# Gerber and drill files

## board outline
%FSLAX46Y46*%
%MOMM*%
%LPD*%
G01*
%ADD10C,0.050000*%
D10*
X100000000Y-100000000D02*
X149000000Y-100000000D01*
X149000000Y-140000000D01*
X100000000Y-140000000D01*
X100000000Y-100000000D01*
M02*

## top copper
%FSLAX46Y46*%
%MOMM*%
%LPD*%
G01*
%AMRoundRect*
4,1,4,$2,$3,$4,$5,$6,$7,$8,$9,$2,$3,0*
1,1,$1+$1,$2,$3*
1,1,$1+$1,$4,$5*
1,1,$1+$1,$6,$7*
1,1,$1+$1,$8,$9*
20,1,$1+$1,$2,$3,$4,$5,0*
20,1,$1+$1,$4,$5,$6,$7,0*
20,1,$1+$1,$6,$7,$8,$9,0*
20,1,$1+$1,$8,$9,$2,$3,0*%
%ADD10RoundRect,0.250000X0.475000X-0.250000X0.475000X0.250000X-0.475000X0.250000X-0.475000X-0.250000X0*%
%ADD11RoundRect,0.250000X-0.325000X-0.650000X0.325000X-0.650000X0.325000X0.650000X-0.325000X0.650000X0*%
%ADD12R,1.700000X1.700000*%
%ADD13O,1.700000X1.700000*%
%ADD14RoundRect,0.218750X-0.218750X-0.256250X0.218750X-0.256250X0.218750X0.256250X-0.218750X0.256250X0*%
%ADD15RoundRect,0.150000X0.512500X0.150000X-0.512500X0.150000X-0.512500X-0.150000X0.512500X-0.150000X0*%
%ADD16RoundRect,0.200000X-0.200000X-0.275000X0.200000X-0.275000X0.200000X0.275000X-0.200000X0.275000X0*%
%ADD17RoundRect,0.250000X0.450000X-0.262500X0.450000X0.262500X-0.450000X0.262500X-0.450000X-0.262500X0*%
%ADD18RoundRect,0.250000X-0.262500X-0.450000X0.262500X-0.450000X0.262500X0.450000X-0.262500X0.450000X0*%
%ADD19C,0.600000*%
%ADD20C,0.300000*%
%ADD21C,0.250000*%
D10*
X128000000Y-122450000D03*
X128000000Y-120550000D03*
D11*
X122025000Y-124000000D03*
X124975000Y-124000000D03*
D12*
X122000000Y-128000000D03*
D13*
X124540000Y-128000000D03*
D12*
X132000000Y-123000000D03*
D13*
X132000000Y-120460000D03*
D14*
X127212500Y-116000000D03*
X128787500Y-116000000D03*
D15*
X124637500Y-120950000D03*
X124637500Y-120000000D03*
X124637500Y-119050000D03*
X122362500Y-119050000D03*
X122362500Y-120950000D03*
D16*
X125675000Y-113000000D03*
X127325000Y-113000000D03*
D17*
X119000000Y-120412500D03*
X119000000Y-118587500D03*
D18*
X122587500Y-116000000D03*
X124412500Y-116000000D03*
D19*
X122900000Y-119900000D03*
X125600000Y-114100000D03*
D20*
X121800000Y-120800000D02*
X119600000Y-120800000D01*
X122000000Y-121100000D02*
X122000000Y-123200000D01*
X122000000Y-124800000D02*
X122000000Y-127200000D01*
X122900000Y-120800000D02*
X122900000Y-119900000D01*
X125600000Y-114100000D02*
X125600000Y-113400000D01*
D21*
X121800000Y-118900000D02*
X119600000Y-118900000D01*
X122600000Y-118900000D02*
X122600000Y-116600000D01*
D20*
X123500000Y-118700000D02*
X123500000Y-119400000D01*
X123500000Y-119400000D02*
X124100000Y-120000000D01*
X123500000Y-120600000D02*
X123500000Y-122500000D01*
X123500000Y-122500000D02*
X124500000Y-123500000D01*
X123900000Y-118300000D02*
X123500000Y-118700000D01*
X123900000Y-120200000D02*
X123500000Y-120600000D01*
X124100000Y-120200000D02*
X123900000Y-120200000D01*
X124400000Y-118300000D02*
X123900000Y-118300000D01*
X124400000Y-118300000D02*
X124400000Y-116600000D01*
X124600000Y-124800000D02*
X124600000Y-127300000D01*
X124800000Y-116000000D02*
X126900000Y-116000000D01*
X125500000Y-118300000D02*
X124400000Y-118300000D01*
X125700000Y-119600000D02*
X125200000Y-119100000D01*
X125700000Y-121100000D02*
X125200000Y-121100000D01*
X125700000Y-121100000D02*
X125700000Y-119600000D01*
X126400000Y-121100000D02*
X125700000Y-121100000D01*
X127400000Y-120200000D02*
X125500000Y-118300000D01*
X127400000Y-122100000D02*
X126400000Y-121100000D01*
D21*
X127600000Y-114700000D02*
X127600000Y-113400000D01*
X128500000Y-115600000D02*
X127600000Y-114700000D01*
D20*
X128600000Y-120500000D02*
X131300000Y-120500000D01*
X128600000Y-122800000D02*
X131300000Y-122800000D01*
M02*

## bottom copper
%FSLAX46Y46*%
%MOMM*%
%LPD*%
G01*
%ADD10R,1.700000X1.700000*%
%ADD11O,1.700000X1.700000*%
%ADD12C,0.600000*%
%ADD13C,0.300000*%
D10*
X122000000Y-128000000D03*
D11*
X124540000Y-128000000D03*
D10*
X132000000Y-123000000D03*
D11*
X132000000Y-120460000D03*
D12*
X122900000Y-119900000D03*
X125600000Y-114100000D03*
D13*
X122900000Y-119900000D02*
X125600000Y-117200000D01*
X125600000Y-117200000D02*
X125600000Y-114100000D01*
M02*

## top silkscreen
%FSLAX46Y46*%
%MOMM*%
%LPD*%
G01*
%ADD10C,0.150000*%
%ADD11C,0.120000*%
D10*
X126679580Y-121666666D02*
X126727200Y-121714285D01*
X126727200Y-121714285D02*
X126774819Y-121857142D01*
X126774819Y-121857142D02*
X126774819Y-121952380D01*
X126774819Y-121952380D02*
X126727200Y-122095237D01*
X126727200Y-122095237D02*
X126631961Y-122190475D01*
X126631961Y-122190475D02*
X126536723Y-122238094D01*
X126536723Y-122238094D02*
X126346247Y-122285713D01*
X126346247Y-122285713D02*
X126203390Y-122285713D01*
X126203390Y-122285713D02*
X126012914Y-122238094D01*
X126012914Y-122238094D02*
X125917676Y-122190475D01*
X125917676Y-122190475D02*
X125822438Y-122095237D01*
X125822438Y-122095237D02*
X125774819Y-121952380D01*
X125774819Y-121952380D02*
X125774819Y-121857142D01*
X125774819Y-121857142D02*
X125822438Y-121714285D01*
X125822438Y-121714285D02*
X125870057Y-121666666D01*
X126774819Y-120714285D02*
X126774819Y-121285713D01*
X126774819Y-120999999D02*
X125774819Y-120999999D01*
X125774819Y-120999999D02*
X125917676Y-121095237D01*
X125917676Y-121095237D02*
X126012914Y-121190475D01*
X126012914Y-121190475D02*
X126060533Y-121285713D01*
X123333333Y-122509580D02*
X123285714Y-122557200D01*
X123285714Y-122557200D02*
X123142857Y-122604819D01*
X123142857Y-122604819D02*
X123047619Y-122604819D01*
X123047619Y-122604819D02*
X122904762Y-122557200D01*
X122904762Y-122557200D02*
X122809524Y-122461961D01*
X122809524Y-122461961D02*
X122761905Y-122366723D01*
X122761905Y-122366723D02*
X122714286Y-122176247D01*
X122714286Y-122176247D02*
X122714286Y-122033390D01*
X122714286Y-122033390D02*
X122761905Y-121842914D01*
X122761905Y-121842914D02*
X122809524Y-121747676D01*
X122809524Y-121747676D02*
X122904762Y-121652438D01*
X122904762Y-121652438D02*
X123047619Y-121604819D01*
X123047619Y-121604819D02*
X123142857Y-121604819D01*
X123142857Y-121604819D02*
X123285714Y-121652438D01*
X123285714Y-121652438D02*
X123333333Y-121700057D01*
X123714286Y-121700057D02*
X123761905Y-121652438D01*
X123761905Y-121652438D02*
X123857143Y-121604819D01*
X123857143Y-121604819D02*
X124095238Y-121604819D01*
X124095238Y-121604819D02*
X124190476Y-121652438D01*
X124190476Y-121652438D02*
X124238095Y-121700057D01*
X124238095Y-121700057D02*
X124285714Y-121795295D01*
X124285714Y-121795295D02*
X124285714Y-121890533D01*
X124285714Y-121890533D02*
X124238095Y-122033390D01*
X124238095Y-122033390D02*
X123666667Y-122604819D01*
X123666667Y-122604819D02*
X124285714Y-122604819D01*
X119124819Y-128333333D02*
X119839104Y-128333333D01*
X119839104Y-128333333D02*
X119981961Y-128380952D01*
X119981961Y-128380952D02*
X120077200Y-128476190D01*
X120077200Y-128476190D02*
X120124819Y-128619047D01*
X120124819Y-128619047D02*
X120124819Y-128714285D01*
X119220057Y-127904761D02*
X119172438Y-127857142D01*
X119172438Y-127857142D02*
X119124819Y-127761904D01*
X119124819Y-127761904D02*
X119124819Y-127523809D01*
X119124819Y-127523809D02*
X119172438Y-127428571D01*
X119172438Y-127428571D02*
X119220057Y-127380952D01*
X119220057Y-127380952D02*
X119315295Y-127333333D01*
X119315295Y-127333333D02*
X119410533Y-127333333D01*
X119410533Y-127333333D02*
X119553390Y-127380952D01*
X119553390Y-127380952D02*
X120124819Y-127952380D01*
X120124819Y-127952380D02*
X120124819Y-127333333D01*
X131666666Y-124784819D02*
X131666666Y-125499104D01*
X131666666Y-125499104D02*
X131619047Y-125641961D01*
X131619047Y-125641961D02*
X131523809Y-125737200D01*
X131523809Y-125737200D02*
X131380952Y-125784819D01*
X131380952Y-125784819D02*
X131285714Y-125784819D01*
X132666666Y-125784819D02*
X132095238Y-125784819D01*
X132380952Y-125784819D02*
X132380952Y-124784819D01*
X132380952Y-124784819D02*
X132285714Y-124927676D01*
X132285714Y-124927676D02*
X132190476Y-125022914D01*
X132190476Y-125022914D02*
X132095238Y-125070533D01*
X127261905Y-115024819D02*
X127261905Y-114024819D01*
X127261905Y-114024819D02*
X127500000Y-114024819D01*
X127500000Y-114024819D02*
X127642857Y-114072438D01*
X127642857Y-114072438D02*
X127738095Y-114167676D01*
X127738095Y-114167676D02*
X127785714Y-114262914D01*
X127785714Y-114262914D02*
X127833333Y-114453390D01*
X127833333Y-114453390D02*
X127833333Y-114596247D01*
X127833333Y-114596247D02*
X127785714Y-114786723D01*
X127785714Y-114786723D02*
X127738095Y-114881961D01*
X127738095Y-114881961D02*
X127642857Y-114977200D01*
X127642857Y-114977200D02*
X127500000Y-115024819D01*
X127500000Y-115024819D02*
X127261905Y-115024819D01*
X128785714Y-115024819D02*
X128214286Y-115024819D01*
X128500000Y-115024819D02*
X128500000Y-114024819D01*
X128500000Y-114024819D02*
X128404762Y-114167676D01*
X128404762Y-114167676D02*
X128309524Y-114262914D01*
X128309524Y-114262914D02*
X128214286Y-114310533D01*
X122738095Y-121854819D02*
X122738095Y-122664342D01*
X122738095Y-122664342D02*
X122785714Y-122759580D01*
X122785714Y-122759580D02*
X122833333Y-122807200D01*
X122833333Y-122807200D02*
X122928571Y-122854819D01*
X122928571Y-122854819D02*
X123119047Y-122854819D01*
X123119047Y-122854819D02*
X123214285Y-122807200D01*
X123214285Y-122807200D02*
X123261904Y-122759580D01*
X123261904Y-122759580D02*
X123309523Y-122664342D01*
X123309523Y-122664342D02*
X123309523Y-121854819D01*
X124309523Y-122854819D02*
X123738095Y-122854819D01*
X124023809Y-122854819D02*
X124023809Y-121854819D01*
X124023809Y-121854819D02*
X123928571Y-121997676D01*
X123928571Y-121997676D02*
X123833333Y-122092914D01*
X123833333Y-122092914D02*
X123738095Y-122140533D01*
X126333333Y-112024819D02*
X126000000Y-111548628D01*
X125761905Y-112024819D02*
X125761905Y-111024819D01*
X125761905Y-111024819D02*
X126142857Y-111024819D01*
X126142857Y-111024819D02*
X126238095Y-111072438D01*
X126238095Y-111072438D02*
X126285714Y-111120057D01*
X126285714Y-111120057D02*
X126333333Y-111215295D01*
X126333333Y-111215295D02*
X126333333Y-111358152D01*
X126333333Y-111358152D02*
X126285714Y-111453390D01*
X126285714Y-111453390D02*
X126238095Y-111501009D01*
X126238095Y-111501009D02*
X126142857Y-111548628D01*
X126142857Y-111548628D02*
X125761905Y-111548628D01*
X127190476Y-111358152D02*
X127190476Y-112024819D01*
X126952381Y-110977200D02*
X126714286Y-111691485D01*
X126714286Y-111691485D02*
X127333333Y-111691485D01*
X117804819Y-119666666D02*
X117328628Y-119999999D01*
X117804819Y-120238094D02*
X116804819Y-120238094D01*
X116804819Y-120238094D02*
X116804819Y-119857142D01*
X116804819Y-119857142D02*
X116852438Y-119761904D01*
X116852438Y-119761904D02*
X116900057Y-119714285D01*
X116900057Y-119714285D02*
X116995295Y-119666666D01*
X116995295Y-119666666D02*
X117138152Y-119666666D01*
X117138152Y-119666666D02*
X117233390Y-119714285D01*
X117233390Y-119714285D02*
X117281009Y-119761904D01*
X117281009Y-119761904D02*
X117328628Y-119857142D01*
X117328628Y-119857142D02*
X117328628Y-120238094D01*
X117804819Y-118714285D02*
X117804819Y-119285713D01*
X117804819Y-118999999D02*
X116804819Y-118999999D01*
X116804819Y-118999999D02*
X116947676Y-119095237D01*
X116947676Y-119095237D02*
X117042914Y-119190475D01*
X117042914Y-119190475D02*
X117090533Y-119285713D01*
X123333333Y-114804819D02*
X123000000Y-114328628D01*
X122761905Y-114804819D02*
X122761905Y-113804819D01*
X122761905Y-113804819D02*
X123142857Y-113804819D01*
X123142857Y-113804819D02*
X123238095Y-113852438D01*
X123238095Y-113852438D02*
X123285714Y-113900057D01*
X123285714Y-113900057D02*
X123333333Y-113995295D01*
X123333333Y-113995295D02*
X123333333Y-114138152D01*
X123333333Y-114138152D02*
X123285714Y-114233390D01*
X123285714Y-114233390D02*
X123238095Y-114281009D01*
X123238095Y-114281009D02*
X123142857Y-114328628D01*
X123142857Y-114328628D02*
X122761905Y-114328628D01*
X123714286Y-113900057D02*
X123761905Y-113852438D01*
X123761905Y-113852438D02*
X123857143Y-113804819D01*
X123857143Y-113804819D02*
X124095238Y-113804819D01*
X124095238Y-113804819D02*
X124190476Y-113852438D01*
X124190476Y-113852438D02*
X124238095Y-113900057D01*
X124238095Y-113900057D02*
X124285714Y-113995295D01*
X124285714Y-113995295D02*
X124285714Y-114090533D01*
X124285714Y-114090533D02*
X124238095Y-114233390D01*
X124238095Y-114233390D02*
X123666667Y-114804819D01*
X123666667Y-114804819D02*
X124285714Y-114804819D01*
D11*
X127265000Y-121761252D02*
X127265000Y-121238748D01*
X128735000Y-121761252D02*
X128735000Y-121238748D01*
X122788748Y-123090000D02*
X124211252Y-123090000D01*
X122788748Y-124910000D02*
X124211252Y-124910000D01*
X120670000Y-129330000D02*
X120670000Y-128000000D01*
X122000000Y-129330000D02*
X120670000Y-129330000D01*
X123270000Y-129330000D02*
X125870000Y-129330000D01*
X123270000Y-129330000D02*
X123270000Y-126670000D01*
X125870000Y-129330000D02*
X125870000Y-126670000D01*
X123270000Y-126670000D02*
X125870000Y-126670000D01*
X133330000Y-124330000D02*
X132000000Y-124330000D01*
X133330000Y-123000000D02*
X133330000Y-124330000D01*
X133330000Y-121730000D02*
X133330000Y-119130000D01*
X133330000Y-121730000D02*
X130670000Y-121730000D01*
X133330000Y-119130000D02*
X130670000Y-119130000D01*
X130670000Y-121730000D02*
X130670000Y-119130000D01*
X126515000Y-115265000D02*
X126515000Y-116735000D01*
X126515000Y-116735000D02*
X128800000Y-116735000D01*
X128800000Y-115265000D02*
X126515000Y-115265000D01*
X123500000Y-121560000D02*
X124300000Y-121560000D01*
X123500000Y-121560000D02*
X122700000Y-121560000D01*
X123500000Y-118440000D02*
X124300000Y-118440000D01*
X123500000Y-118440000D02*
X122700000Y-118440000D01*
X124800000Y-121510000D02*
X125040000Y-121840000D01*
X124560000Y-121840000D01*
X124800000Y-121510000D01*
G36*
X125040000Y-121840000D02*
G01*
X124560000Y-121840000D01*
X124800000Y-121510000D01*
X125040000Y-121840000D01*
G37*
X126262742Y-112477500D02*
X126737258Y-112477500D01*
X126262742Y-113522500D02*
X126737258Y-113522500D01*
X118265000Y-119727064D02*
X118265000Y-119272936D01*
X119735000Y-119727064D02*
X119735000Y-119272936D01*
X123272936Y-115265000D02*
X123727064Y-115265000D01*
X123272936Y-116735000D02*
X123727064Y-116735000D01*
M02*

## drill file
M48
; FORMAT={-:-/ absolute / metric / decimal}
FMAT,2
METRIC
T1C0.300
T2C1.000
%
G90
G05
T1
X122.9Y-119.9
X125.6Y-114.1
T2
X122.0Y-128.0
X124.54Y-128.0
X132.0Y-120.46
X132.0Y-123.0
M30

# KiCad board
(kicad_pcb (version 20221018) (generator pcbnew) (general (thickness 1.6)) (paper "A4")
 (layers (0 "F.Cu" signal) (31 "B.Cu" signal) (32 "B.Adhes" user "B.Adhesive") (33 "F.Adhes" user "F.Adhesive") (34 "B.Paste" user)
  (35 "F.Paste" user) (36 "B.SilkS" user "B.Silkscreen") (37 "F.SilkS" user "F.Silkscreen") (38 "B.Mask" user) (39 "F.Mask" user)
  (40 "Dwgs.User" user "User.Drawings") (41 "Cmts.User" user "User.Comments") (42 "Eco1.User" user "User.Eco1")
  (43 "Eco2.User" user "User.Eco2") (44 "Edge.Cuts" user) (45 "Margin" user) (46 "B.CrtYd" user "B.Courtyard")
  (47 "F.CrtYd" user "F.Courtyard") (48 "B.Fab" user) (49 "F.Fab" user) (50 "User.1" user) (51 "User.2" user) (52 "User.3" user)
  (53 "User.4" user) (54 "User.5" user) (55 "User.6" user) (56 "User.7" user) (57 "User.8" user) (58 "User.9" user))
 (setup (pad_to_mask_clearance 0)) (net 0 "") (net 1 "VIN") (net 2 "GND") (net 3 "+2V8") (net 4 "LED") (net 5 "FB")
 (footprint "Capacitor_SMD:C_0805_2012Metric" (layer "F.Cu") (at 128 121.5 90)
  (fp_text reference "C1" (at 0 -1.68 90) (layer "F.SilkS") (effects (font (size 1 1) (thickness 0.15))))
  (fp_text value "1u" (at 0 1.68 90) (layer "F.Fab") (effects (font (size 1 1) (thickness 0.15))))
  (fp_line (start -0.261252 -0.735) (end 0.261252 -0.735) (stroke (width 0.12) (type solid)) (layer "F.SilkS"))
  (fp_line (start -0.261252 0.735) (end 0.261252 0.735) (stroke (width 0.12) (type solid)) (layer "F.SilkS"))
  (pad "1" smd roundrect (at -0.95 0 90) (size 1 1.45) (layers "F.Cu" "F.Paste" "F.Mask") (roundrect_rratio 0.25) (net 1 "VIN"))
  (pad "2" smd roundrect (at 0.95 0 90) (size 1 1.45) (layers "F.Cu" "F.Paste" "F.Mask") (roundrect_rratio 0.25) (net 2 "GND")))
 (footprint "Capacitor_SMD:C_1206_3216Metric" (layer "F.Cu") (at 123.5 124)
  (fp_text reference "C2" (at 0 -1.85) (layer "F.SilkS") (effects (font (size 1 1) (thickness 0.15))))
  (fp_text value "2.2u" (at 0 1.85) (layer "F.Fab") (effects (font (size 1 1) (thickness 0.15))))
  (fp_line (start -0.711252 -0.91) (end 0.711252 -0.91) (stroke (width 0.12) (type solid)) (layer "F.SilkS"))
  (fp_line (start -0.711252 0.91) (end 0.711252 0.91) (stroke (width 0.12) (type solid)) (layer "F.SilkS"))
  (pad "1" smd roundrect (at -1.475 0) (size 1.15 1.8) (layers "F.Cu" "F.Paste" "F.Mask") (roundrect_rratio 0.217391) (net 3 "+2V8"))
  (pad "2" smd roundrect (at 1.475 0) (size 1.15 1.8) (layers "F.Cu" "F.Paste" "F.Mask") (roundrect_rratio 0.217391) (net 2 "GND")))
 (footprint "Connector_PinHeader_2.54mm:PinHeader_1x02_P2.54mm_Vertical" (layer "F.Cu") (at 122 128 90)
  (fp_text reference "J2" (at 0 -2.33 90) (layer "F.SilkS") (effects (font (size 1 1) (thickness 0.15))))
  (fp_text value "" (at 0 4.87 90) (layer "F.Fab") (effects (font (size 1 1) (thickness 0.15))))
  (fp_line (start -1.33 -1.33) (end 0 -1.33) (stroke (width 0.12) (type solid)) (layer "F.SilkS"))
  (fp_line (start -1.33 0) (end -1.33 -1.33) (stroke (width 0.12) (type solid)) (layer "F.SilkS"))
  (fp_line (start -1.33 1.27) (end -1.33 3.87) (stroke (width 0.12) (type solid)) (layer "F.SilkS"))
  (fp_line (start -1.33 1.27) (end 1.33 1.27) (stroke (width 0.12) (type solid)) (layer "F.SilkS"))
  (fp_line (start -1.33 3.87) (end 1.33 3.87) (stroke (width 0.12) (type solid)) (layer "F.SilkS"))
  (fp_line (start 1.33 1.27) (end 1.33 3.87) (stroke (width 0.12) (type solid)) (layer "F.SilkS"))
  (pad "1" thru_hole rect (at 0 0 90) (size 1.7 1.7) (drill 1) (layers "*.Cu" "*.Mask") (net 3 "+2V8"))
  (pad "2" thru_hole oval (at 0 2.54 90) (size 1.7 1.7) (drill 1) (layers "*.Cu" "*.Mask") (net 2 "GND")))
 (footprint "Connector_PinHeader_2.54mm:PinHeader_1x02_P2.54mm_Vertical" (layer "F.Cu") (at 132 123 180)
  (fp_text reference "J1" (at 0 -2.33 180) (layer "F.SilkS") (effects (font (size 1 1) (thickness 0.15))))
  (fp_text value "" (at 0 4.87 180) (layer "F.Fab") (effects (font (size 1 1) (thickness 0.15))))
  (fp_line (start -1.33 -1.33) (end 0 -1.33) (stroke (width 0.12) (type solid)) (layer "F.SilkS"))
  (fp_line (start -1.33 0) (end -1.33 -1.33) (stroke (width 0.12) (type solid)) (layer "F.SilkS"))
  (fp_line (start -1.33 1.27) (end -1.33 3.87) (stroke (width 0.12) (type solid)) (layer "F.SilkS"))
  (fp_line (start -1.33 1.27) (end 1.33 1.27) (stroke (width 0.12) (type solid)) (layer "F.SilkS"))
  (fp_line (start -1.33 3.87) (end 1.33 3.87) (stroke (width 0.12) (type solid)) (layer "F.SilkS"))
  (fp_line (start 1.33 1.27) (end 1.33 3.87) (stroke (width 0.12) (type solid)) (layer "F.SilkS"))
  (pad "1" thru_hole rect (at 0 0 180) (size 1.7 1.7) (drill 1) (layers "*.Cu" "*.Mask") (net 1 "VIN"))
  (pad "2" thru_hole oval (at 0 2.54 180) (size 1.7 1.7) (drill 1) (layers "*.Cu" "*.Mask") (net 2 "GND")))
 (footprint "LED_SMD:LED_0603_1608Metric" (layer "F.Cu") (at 128 116)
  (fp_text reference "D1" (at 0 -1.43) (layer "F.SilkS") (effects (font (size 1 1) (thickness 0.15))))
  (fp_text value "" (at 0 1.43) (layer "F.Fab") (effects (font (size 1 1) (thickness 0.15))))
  (fp_line (start -1.485 -0.735) (end -1.485 0.735) (stroke (width 0.12) (type solid)) (layer "F.SilkS"))
  (fp_line (start -1.485 0.735) (end 0.8 0.735) (stroke (width 0.12) (type solid)) (layer "F.SilkS"))
  (fp_line (start 0.8 -0.735) (end -1.485 -0.735) (stroke (width 0.12) (type solid)) (layer "F.SilkS"))
  (pad "1" smd roundrect (at -0.7875 0) (size 0.875 0.95) (layers "F.Cu" "F.Paste" "F.Mask") (roundrect_rratio 0.25) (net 2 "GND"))
  (pad "2" smd roundrect (at 0.7875 0) (size 0.875 0.95) (layers "F.Cu" "F.Paste" "F.Mask") (roundrect_rratio 0.25) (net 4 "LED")))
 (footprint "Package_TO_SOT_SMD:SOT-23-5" (layer "F.Cu") (at 123.5 120 180)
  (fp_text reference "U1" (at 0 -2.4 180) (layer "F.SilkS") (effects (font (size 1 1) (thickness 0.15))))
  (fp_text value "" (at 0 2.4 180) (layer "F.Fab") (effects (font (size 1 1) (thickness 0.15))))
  (fp_line (start 0 -1.56) (end -0.8 -1.56) (stroke (width 0.12) (type solid)) (layer "F.SilkS"))
  (fp_line (start 0 -1.56) (end 0.8 -1.56) (stroke (width 0.12) (type solid)) (layer "F.SilkS"))
  (fp_line (start 0 1.56) (end -0.8 1.56) (stroke (width 0.12) (type solid)) (layer "F.SilkS"))
  (fp_line (start 0 1.56) (end 0.8 1.56) (stroke (width 0.12) (type solid)) (layer "F.SilkS"))
  (fp_poly
   (pts (xy -1.3 -1.51) (xy -1.54 -1.84) (xy -1.06 -1.84) (xy -1.3 -1.51)) (stroke (width 0.12) (type solid)) (fill solid) (layer "F.SilkS"))
  (pad "1" smd roundrect (at -1.1375 -0.95 180) (size 1.325 0.6) (layers "F.Cu" "F.Paste" "F.Mask") (roundrect_rratio 0.25) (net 1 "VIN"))
  (pad "2" smd roundrect (at -1.1375 0 180) (size 1.325 0.6) (layers "F.Cu" "F.Paste" "F.Mask") (roundrect_rratio 0.25) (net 2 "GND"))
  (pad "3" smd roundrect (at -1.1375 0.95 180) (size 1.325 0.6) (layers "F.Cu" "F.Paste" "F.Mask") (roundrect_rratio 0.25) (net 1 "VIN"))
  (pad "4" smd roundrect (at 1.1375 0.95 180) (size 1.325 0.6) (layers "F.Cu" "F.Paste" "F.Mask") (roundrect_rratio 0.25) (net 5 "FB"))
  (pad "5" smd roundrect (at 1.1375 -0.95 180) (size 1.325 0.6) (layers "F.Cu" "F.Paste" "F.Mask") (roundrect_rratio 0.25) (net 3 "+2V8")))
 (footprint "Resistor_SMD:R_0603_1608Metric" (layer "F.Cu") (at 126.5 113)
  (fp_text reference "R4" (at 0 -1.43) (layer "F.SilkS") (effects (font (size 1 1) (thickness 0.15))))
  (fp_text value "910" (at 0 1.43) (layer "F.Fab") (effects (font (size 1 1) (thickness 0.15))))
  (fp_line (start -0.237258 -0.5225) (end 0.237258 -0.5225) (stroke (width 0.12) (type solid)) (layer "F.SilkS"))
  (fp_line (start -0.237258 0.5225) (end 0.237258 0.5225) (stroke (width 0.12) (type solid)) (layer "F.SilkS"))
  (pad "1" smd roundrect (at -0.825 0) (size 0.8 0.95) (layers "F.Cu" "F.Paste" "F.Mask") (roundrect_rratio 0.25) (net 3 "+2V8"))
  (pad "2" smd roundrect (at 0.825 0) (size 0.8 0.95) (layers "F.Cu" "F.Paste" "F.Mask") (roundrect_rratio 0.25) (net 4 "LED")))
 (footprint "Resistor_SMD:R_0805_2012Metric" (layer "F.Cu") (at 119 119.5 90)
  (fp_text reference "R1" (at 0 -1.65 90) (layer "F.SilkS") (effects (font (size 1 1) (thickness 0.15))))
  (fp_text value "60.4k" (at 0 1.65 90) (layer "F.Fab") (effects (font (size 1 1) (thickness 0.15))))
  (fp_line (start -0.227064 -0.735) (end 0.227064 -0.735) (stroke (width 0.12) (type solid)) (layer "F.SilkS"))
  (fp_line (start -0.227064 0.735) (end 0.227064 0.735) (stroke (width 0.12) (type solid)) (layer "F.SilkS"))
  (pad "1" smd roundrect (at -0.9125 0 90) (size 1.025 1.4) (layers "F.Cu" "F.Paste" "F.Mask") (roundrect_rratio 0.243902) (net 3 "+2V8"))
  (pad "2" smd roundrect (at 0.9125 0 90) (size 1.025 1.4) (layers "F.Cu" "F.Paste" "F.Mask") (roundrect_rratio 0.243902) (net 5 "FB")))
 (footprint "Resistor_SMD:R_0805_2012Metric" (layer "F.Cu") (at 123.5 116)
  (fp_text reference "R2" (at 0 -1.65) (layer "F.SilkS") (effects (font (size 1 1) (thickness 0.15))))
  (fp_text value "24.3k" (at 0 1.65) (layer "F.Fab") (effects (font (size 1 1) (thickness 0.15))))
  (fp_line (start -0.227064 -0.735) (end 0.227064 -0.735) (stroke (width 0.12) (type solid)) (layer "F.SilkS"))
  (fp_line (start -0.227064 0.735) (end 0.227064 0.735) (stroke (width 0.12) (type solid)) (layer "F.SilkS"))
  (pad "1" smd roundrect (at -0.9125 0) (size 1.025 1.4) (layers "F.Cu" "F.Paste" "F.Mask") (roundrect_rratio 0.243902) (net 5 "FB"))
  (pad "2" smd roundrect (at 0.9125 0) (size 1.025 1.4) (layers "F.Cu" "F.Paste" "F.Mask") (roundrect_rratio 0.243902) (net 2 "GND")))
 (gr_rect (start 100 100) (end 149 140) (stroke (width 0.05) (type default)) (fill none) (layer "Edge.Cuts"))
 (segment (start 121.8 120.8) (end 119.6 120.8) (width 0.3) (layer "F.Cu") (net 3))
 (segment (start 122 121.1) (end 122 123.2) (width 0.3) (layer "F.Cu") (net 3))
 (segment (start 122 124.8) (end 122 127.2) (width 0.3) (layer "F.Cu") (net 3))
 (segment (start 122.9 120.8) (end 122.9 119.9) (width 0.3) (layer "F.Cu") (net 3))
 (segment (start 125.6 114.1) (end 125.6 113.4) (width 0.3) (layer "F.Cu") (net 3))
 (via (at 122.9 119.9) (size 0.6) (drill 0.3) (layers "F.Cu" "B.Cu") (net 3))
 (via (at 125.6 114.1) (size 0.6) (drill 0.3) (layers "F.Cu" "B.Cu") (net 3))
 (segment (start 121.8 118.9) (end 119.6 118.9) (width 0.25) (layer "F.Cu") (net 5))
 (segment (start 122.6 118.9) (end 122.6 116.6) (width 0.25) (layer "F.Cu") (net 5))
 (segment (start 122.9 119.9) (end 125.6 117.2) (width 0.3) (layer "B.Cu") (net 3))
 (segment (start 123.5 118.7) (end 123.5 119.4) (width 0.3) (layer "F.Cu") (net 2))
 (segment (start 123.5 119.4) (end 124.1 120) (width 0.3) (layer "F.Cu") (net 2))
 (segment (start 123.5 120.6) (end 123.5 122.5) (width 0.3) (layer "F.Cu") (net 2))
 (segment (start 123.5 122.5) (end 124.5 123.5) (width 0.3) (layer "F.Cu") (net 2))
 (segment (start 123.9 118.3) (end 123.5 118.7) (width 0.3) (layer "F.Cu") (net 2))
 (segment (start 123.9 120.2) (end 123.5 120.6) (width 0.3) (layer "F.Cu") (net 2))
 (segment (start 124.1 120.2) (end 123.9 120.2) (width 0.3) (layer "F.Cu") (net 2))
 (segment (start 124.4 118.3) (end 123.9 118.3) (width 0.3) (layer "F.Cu") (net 2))
 (segment (start 124.4 118.3) (end 124.4 116.6) (width 0.3) (layer "F.Cu") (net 2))
 (segment (start 124.6 124.8) (end 124.6 127.3) (width 0.3) (layer "F.Cu") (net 2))
 (segment (start 124.8 116) (end 126.9 116) (width 0.3) (layer "F.Cu") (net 2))
 (segment (start 125.5 118.3) (end 124.4 118.3) (width 0.3) (layer "F.Cu") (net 2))
 (segment (start 125.6 117.2) (end 125.6 114.1) (width 0.3) (layer "B.Cu") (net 3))
 (segment (start 125.7 119.6) (end 125.2 119.1) (width 0.3) (layer "F.Cu") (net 1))
 (segment (start 125.7 121.1) (end 125.2 121.1) (width 0.3) (layer "F.Cu") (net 1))
 (segment (start 125.7 121.1) (end 125.7 119.6) (width 0.3) (layer "F.Cu") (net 1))
 (segment (start 126.4 121.1) (end 125.7 121.1) (width 0.3) (layer "F.Cu") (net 1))
 (segment (start 127.4 120.2) (end 125.5 118.3) (width 0.3) (layer "F.Cu") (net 2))
 (segment (start 127.4 122.1) (end 126.4 121.1) (width 0.3) (layer "F.Cu") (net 1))
 (segment (start 127.6 114.7) (end 127.6 113.4) (width 0.25) (layer "F.Cu") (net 4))
 (segment (start 128.5 115.6) (end 127.6 114.7) (width 0.25) (layer "F.Cu") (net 4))
 (segment (start 128.6 120.5) (end 131.3 120.5) (width 0.3) (layer "F.Cu") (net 2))
 (segment (start 128.6 122.8) (end 131.3 122.8) (width 0.3) (layer "F.Cu") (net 1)))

